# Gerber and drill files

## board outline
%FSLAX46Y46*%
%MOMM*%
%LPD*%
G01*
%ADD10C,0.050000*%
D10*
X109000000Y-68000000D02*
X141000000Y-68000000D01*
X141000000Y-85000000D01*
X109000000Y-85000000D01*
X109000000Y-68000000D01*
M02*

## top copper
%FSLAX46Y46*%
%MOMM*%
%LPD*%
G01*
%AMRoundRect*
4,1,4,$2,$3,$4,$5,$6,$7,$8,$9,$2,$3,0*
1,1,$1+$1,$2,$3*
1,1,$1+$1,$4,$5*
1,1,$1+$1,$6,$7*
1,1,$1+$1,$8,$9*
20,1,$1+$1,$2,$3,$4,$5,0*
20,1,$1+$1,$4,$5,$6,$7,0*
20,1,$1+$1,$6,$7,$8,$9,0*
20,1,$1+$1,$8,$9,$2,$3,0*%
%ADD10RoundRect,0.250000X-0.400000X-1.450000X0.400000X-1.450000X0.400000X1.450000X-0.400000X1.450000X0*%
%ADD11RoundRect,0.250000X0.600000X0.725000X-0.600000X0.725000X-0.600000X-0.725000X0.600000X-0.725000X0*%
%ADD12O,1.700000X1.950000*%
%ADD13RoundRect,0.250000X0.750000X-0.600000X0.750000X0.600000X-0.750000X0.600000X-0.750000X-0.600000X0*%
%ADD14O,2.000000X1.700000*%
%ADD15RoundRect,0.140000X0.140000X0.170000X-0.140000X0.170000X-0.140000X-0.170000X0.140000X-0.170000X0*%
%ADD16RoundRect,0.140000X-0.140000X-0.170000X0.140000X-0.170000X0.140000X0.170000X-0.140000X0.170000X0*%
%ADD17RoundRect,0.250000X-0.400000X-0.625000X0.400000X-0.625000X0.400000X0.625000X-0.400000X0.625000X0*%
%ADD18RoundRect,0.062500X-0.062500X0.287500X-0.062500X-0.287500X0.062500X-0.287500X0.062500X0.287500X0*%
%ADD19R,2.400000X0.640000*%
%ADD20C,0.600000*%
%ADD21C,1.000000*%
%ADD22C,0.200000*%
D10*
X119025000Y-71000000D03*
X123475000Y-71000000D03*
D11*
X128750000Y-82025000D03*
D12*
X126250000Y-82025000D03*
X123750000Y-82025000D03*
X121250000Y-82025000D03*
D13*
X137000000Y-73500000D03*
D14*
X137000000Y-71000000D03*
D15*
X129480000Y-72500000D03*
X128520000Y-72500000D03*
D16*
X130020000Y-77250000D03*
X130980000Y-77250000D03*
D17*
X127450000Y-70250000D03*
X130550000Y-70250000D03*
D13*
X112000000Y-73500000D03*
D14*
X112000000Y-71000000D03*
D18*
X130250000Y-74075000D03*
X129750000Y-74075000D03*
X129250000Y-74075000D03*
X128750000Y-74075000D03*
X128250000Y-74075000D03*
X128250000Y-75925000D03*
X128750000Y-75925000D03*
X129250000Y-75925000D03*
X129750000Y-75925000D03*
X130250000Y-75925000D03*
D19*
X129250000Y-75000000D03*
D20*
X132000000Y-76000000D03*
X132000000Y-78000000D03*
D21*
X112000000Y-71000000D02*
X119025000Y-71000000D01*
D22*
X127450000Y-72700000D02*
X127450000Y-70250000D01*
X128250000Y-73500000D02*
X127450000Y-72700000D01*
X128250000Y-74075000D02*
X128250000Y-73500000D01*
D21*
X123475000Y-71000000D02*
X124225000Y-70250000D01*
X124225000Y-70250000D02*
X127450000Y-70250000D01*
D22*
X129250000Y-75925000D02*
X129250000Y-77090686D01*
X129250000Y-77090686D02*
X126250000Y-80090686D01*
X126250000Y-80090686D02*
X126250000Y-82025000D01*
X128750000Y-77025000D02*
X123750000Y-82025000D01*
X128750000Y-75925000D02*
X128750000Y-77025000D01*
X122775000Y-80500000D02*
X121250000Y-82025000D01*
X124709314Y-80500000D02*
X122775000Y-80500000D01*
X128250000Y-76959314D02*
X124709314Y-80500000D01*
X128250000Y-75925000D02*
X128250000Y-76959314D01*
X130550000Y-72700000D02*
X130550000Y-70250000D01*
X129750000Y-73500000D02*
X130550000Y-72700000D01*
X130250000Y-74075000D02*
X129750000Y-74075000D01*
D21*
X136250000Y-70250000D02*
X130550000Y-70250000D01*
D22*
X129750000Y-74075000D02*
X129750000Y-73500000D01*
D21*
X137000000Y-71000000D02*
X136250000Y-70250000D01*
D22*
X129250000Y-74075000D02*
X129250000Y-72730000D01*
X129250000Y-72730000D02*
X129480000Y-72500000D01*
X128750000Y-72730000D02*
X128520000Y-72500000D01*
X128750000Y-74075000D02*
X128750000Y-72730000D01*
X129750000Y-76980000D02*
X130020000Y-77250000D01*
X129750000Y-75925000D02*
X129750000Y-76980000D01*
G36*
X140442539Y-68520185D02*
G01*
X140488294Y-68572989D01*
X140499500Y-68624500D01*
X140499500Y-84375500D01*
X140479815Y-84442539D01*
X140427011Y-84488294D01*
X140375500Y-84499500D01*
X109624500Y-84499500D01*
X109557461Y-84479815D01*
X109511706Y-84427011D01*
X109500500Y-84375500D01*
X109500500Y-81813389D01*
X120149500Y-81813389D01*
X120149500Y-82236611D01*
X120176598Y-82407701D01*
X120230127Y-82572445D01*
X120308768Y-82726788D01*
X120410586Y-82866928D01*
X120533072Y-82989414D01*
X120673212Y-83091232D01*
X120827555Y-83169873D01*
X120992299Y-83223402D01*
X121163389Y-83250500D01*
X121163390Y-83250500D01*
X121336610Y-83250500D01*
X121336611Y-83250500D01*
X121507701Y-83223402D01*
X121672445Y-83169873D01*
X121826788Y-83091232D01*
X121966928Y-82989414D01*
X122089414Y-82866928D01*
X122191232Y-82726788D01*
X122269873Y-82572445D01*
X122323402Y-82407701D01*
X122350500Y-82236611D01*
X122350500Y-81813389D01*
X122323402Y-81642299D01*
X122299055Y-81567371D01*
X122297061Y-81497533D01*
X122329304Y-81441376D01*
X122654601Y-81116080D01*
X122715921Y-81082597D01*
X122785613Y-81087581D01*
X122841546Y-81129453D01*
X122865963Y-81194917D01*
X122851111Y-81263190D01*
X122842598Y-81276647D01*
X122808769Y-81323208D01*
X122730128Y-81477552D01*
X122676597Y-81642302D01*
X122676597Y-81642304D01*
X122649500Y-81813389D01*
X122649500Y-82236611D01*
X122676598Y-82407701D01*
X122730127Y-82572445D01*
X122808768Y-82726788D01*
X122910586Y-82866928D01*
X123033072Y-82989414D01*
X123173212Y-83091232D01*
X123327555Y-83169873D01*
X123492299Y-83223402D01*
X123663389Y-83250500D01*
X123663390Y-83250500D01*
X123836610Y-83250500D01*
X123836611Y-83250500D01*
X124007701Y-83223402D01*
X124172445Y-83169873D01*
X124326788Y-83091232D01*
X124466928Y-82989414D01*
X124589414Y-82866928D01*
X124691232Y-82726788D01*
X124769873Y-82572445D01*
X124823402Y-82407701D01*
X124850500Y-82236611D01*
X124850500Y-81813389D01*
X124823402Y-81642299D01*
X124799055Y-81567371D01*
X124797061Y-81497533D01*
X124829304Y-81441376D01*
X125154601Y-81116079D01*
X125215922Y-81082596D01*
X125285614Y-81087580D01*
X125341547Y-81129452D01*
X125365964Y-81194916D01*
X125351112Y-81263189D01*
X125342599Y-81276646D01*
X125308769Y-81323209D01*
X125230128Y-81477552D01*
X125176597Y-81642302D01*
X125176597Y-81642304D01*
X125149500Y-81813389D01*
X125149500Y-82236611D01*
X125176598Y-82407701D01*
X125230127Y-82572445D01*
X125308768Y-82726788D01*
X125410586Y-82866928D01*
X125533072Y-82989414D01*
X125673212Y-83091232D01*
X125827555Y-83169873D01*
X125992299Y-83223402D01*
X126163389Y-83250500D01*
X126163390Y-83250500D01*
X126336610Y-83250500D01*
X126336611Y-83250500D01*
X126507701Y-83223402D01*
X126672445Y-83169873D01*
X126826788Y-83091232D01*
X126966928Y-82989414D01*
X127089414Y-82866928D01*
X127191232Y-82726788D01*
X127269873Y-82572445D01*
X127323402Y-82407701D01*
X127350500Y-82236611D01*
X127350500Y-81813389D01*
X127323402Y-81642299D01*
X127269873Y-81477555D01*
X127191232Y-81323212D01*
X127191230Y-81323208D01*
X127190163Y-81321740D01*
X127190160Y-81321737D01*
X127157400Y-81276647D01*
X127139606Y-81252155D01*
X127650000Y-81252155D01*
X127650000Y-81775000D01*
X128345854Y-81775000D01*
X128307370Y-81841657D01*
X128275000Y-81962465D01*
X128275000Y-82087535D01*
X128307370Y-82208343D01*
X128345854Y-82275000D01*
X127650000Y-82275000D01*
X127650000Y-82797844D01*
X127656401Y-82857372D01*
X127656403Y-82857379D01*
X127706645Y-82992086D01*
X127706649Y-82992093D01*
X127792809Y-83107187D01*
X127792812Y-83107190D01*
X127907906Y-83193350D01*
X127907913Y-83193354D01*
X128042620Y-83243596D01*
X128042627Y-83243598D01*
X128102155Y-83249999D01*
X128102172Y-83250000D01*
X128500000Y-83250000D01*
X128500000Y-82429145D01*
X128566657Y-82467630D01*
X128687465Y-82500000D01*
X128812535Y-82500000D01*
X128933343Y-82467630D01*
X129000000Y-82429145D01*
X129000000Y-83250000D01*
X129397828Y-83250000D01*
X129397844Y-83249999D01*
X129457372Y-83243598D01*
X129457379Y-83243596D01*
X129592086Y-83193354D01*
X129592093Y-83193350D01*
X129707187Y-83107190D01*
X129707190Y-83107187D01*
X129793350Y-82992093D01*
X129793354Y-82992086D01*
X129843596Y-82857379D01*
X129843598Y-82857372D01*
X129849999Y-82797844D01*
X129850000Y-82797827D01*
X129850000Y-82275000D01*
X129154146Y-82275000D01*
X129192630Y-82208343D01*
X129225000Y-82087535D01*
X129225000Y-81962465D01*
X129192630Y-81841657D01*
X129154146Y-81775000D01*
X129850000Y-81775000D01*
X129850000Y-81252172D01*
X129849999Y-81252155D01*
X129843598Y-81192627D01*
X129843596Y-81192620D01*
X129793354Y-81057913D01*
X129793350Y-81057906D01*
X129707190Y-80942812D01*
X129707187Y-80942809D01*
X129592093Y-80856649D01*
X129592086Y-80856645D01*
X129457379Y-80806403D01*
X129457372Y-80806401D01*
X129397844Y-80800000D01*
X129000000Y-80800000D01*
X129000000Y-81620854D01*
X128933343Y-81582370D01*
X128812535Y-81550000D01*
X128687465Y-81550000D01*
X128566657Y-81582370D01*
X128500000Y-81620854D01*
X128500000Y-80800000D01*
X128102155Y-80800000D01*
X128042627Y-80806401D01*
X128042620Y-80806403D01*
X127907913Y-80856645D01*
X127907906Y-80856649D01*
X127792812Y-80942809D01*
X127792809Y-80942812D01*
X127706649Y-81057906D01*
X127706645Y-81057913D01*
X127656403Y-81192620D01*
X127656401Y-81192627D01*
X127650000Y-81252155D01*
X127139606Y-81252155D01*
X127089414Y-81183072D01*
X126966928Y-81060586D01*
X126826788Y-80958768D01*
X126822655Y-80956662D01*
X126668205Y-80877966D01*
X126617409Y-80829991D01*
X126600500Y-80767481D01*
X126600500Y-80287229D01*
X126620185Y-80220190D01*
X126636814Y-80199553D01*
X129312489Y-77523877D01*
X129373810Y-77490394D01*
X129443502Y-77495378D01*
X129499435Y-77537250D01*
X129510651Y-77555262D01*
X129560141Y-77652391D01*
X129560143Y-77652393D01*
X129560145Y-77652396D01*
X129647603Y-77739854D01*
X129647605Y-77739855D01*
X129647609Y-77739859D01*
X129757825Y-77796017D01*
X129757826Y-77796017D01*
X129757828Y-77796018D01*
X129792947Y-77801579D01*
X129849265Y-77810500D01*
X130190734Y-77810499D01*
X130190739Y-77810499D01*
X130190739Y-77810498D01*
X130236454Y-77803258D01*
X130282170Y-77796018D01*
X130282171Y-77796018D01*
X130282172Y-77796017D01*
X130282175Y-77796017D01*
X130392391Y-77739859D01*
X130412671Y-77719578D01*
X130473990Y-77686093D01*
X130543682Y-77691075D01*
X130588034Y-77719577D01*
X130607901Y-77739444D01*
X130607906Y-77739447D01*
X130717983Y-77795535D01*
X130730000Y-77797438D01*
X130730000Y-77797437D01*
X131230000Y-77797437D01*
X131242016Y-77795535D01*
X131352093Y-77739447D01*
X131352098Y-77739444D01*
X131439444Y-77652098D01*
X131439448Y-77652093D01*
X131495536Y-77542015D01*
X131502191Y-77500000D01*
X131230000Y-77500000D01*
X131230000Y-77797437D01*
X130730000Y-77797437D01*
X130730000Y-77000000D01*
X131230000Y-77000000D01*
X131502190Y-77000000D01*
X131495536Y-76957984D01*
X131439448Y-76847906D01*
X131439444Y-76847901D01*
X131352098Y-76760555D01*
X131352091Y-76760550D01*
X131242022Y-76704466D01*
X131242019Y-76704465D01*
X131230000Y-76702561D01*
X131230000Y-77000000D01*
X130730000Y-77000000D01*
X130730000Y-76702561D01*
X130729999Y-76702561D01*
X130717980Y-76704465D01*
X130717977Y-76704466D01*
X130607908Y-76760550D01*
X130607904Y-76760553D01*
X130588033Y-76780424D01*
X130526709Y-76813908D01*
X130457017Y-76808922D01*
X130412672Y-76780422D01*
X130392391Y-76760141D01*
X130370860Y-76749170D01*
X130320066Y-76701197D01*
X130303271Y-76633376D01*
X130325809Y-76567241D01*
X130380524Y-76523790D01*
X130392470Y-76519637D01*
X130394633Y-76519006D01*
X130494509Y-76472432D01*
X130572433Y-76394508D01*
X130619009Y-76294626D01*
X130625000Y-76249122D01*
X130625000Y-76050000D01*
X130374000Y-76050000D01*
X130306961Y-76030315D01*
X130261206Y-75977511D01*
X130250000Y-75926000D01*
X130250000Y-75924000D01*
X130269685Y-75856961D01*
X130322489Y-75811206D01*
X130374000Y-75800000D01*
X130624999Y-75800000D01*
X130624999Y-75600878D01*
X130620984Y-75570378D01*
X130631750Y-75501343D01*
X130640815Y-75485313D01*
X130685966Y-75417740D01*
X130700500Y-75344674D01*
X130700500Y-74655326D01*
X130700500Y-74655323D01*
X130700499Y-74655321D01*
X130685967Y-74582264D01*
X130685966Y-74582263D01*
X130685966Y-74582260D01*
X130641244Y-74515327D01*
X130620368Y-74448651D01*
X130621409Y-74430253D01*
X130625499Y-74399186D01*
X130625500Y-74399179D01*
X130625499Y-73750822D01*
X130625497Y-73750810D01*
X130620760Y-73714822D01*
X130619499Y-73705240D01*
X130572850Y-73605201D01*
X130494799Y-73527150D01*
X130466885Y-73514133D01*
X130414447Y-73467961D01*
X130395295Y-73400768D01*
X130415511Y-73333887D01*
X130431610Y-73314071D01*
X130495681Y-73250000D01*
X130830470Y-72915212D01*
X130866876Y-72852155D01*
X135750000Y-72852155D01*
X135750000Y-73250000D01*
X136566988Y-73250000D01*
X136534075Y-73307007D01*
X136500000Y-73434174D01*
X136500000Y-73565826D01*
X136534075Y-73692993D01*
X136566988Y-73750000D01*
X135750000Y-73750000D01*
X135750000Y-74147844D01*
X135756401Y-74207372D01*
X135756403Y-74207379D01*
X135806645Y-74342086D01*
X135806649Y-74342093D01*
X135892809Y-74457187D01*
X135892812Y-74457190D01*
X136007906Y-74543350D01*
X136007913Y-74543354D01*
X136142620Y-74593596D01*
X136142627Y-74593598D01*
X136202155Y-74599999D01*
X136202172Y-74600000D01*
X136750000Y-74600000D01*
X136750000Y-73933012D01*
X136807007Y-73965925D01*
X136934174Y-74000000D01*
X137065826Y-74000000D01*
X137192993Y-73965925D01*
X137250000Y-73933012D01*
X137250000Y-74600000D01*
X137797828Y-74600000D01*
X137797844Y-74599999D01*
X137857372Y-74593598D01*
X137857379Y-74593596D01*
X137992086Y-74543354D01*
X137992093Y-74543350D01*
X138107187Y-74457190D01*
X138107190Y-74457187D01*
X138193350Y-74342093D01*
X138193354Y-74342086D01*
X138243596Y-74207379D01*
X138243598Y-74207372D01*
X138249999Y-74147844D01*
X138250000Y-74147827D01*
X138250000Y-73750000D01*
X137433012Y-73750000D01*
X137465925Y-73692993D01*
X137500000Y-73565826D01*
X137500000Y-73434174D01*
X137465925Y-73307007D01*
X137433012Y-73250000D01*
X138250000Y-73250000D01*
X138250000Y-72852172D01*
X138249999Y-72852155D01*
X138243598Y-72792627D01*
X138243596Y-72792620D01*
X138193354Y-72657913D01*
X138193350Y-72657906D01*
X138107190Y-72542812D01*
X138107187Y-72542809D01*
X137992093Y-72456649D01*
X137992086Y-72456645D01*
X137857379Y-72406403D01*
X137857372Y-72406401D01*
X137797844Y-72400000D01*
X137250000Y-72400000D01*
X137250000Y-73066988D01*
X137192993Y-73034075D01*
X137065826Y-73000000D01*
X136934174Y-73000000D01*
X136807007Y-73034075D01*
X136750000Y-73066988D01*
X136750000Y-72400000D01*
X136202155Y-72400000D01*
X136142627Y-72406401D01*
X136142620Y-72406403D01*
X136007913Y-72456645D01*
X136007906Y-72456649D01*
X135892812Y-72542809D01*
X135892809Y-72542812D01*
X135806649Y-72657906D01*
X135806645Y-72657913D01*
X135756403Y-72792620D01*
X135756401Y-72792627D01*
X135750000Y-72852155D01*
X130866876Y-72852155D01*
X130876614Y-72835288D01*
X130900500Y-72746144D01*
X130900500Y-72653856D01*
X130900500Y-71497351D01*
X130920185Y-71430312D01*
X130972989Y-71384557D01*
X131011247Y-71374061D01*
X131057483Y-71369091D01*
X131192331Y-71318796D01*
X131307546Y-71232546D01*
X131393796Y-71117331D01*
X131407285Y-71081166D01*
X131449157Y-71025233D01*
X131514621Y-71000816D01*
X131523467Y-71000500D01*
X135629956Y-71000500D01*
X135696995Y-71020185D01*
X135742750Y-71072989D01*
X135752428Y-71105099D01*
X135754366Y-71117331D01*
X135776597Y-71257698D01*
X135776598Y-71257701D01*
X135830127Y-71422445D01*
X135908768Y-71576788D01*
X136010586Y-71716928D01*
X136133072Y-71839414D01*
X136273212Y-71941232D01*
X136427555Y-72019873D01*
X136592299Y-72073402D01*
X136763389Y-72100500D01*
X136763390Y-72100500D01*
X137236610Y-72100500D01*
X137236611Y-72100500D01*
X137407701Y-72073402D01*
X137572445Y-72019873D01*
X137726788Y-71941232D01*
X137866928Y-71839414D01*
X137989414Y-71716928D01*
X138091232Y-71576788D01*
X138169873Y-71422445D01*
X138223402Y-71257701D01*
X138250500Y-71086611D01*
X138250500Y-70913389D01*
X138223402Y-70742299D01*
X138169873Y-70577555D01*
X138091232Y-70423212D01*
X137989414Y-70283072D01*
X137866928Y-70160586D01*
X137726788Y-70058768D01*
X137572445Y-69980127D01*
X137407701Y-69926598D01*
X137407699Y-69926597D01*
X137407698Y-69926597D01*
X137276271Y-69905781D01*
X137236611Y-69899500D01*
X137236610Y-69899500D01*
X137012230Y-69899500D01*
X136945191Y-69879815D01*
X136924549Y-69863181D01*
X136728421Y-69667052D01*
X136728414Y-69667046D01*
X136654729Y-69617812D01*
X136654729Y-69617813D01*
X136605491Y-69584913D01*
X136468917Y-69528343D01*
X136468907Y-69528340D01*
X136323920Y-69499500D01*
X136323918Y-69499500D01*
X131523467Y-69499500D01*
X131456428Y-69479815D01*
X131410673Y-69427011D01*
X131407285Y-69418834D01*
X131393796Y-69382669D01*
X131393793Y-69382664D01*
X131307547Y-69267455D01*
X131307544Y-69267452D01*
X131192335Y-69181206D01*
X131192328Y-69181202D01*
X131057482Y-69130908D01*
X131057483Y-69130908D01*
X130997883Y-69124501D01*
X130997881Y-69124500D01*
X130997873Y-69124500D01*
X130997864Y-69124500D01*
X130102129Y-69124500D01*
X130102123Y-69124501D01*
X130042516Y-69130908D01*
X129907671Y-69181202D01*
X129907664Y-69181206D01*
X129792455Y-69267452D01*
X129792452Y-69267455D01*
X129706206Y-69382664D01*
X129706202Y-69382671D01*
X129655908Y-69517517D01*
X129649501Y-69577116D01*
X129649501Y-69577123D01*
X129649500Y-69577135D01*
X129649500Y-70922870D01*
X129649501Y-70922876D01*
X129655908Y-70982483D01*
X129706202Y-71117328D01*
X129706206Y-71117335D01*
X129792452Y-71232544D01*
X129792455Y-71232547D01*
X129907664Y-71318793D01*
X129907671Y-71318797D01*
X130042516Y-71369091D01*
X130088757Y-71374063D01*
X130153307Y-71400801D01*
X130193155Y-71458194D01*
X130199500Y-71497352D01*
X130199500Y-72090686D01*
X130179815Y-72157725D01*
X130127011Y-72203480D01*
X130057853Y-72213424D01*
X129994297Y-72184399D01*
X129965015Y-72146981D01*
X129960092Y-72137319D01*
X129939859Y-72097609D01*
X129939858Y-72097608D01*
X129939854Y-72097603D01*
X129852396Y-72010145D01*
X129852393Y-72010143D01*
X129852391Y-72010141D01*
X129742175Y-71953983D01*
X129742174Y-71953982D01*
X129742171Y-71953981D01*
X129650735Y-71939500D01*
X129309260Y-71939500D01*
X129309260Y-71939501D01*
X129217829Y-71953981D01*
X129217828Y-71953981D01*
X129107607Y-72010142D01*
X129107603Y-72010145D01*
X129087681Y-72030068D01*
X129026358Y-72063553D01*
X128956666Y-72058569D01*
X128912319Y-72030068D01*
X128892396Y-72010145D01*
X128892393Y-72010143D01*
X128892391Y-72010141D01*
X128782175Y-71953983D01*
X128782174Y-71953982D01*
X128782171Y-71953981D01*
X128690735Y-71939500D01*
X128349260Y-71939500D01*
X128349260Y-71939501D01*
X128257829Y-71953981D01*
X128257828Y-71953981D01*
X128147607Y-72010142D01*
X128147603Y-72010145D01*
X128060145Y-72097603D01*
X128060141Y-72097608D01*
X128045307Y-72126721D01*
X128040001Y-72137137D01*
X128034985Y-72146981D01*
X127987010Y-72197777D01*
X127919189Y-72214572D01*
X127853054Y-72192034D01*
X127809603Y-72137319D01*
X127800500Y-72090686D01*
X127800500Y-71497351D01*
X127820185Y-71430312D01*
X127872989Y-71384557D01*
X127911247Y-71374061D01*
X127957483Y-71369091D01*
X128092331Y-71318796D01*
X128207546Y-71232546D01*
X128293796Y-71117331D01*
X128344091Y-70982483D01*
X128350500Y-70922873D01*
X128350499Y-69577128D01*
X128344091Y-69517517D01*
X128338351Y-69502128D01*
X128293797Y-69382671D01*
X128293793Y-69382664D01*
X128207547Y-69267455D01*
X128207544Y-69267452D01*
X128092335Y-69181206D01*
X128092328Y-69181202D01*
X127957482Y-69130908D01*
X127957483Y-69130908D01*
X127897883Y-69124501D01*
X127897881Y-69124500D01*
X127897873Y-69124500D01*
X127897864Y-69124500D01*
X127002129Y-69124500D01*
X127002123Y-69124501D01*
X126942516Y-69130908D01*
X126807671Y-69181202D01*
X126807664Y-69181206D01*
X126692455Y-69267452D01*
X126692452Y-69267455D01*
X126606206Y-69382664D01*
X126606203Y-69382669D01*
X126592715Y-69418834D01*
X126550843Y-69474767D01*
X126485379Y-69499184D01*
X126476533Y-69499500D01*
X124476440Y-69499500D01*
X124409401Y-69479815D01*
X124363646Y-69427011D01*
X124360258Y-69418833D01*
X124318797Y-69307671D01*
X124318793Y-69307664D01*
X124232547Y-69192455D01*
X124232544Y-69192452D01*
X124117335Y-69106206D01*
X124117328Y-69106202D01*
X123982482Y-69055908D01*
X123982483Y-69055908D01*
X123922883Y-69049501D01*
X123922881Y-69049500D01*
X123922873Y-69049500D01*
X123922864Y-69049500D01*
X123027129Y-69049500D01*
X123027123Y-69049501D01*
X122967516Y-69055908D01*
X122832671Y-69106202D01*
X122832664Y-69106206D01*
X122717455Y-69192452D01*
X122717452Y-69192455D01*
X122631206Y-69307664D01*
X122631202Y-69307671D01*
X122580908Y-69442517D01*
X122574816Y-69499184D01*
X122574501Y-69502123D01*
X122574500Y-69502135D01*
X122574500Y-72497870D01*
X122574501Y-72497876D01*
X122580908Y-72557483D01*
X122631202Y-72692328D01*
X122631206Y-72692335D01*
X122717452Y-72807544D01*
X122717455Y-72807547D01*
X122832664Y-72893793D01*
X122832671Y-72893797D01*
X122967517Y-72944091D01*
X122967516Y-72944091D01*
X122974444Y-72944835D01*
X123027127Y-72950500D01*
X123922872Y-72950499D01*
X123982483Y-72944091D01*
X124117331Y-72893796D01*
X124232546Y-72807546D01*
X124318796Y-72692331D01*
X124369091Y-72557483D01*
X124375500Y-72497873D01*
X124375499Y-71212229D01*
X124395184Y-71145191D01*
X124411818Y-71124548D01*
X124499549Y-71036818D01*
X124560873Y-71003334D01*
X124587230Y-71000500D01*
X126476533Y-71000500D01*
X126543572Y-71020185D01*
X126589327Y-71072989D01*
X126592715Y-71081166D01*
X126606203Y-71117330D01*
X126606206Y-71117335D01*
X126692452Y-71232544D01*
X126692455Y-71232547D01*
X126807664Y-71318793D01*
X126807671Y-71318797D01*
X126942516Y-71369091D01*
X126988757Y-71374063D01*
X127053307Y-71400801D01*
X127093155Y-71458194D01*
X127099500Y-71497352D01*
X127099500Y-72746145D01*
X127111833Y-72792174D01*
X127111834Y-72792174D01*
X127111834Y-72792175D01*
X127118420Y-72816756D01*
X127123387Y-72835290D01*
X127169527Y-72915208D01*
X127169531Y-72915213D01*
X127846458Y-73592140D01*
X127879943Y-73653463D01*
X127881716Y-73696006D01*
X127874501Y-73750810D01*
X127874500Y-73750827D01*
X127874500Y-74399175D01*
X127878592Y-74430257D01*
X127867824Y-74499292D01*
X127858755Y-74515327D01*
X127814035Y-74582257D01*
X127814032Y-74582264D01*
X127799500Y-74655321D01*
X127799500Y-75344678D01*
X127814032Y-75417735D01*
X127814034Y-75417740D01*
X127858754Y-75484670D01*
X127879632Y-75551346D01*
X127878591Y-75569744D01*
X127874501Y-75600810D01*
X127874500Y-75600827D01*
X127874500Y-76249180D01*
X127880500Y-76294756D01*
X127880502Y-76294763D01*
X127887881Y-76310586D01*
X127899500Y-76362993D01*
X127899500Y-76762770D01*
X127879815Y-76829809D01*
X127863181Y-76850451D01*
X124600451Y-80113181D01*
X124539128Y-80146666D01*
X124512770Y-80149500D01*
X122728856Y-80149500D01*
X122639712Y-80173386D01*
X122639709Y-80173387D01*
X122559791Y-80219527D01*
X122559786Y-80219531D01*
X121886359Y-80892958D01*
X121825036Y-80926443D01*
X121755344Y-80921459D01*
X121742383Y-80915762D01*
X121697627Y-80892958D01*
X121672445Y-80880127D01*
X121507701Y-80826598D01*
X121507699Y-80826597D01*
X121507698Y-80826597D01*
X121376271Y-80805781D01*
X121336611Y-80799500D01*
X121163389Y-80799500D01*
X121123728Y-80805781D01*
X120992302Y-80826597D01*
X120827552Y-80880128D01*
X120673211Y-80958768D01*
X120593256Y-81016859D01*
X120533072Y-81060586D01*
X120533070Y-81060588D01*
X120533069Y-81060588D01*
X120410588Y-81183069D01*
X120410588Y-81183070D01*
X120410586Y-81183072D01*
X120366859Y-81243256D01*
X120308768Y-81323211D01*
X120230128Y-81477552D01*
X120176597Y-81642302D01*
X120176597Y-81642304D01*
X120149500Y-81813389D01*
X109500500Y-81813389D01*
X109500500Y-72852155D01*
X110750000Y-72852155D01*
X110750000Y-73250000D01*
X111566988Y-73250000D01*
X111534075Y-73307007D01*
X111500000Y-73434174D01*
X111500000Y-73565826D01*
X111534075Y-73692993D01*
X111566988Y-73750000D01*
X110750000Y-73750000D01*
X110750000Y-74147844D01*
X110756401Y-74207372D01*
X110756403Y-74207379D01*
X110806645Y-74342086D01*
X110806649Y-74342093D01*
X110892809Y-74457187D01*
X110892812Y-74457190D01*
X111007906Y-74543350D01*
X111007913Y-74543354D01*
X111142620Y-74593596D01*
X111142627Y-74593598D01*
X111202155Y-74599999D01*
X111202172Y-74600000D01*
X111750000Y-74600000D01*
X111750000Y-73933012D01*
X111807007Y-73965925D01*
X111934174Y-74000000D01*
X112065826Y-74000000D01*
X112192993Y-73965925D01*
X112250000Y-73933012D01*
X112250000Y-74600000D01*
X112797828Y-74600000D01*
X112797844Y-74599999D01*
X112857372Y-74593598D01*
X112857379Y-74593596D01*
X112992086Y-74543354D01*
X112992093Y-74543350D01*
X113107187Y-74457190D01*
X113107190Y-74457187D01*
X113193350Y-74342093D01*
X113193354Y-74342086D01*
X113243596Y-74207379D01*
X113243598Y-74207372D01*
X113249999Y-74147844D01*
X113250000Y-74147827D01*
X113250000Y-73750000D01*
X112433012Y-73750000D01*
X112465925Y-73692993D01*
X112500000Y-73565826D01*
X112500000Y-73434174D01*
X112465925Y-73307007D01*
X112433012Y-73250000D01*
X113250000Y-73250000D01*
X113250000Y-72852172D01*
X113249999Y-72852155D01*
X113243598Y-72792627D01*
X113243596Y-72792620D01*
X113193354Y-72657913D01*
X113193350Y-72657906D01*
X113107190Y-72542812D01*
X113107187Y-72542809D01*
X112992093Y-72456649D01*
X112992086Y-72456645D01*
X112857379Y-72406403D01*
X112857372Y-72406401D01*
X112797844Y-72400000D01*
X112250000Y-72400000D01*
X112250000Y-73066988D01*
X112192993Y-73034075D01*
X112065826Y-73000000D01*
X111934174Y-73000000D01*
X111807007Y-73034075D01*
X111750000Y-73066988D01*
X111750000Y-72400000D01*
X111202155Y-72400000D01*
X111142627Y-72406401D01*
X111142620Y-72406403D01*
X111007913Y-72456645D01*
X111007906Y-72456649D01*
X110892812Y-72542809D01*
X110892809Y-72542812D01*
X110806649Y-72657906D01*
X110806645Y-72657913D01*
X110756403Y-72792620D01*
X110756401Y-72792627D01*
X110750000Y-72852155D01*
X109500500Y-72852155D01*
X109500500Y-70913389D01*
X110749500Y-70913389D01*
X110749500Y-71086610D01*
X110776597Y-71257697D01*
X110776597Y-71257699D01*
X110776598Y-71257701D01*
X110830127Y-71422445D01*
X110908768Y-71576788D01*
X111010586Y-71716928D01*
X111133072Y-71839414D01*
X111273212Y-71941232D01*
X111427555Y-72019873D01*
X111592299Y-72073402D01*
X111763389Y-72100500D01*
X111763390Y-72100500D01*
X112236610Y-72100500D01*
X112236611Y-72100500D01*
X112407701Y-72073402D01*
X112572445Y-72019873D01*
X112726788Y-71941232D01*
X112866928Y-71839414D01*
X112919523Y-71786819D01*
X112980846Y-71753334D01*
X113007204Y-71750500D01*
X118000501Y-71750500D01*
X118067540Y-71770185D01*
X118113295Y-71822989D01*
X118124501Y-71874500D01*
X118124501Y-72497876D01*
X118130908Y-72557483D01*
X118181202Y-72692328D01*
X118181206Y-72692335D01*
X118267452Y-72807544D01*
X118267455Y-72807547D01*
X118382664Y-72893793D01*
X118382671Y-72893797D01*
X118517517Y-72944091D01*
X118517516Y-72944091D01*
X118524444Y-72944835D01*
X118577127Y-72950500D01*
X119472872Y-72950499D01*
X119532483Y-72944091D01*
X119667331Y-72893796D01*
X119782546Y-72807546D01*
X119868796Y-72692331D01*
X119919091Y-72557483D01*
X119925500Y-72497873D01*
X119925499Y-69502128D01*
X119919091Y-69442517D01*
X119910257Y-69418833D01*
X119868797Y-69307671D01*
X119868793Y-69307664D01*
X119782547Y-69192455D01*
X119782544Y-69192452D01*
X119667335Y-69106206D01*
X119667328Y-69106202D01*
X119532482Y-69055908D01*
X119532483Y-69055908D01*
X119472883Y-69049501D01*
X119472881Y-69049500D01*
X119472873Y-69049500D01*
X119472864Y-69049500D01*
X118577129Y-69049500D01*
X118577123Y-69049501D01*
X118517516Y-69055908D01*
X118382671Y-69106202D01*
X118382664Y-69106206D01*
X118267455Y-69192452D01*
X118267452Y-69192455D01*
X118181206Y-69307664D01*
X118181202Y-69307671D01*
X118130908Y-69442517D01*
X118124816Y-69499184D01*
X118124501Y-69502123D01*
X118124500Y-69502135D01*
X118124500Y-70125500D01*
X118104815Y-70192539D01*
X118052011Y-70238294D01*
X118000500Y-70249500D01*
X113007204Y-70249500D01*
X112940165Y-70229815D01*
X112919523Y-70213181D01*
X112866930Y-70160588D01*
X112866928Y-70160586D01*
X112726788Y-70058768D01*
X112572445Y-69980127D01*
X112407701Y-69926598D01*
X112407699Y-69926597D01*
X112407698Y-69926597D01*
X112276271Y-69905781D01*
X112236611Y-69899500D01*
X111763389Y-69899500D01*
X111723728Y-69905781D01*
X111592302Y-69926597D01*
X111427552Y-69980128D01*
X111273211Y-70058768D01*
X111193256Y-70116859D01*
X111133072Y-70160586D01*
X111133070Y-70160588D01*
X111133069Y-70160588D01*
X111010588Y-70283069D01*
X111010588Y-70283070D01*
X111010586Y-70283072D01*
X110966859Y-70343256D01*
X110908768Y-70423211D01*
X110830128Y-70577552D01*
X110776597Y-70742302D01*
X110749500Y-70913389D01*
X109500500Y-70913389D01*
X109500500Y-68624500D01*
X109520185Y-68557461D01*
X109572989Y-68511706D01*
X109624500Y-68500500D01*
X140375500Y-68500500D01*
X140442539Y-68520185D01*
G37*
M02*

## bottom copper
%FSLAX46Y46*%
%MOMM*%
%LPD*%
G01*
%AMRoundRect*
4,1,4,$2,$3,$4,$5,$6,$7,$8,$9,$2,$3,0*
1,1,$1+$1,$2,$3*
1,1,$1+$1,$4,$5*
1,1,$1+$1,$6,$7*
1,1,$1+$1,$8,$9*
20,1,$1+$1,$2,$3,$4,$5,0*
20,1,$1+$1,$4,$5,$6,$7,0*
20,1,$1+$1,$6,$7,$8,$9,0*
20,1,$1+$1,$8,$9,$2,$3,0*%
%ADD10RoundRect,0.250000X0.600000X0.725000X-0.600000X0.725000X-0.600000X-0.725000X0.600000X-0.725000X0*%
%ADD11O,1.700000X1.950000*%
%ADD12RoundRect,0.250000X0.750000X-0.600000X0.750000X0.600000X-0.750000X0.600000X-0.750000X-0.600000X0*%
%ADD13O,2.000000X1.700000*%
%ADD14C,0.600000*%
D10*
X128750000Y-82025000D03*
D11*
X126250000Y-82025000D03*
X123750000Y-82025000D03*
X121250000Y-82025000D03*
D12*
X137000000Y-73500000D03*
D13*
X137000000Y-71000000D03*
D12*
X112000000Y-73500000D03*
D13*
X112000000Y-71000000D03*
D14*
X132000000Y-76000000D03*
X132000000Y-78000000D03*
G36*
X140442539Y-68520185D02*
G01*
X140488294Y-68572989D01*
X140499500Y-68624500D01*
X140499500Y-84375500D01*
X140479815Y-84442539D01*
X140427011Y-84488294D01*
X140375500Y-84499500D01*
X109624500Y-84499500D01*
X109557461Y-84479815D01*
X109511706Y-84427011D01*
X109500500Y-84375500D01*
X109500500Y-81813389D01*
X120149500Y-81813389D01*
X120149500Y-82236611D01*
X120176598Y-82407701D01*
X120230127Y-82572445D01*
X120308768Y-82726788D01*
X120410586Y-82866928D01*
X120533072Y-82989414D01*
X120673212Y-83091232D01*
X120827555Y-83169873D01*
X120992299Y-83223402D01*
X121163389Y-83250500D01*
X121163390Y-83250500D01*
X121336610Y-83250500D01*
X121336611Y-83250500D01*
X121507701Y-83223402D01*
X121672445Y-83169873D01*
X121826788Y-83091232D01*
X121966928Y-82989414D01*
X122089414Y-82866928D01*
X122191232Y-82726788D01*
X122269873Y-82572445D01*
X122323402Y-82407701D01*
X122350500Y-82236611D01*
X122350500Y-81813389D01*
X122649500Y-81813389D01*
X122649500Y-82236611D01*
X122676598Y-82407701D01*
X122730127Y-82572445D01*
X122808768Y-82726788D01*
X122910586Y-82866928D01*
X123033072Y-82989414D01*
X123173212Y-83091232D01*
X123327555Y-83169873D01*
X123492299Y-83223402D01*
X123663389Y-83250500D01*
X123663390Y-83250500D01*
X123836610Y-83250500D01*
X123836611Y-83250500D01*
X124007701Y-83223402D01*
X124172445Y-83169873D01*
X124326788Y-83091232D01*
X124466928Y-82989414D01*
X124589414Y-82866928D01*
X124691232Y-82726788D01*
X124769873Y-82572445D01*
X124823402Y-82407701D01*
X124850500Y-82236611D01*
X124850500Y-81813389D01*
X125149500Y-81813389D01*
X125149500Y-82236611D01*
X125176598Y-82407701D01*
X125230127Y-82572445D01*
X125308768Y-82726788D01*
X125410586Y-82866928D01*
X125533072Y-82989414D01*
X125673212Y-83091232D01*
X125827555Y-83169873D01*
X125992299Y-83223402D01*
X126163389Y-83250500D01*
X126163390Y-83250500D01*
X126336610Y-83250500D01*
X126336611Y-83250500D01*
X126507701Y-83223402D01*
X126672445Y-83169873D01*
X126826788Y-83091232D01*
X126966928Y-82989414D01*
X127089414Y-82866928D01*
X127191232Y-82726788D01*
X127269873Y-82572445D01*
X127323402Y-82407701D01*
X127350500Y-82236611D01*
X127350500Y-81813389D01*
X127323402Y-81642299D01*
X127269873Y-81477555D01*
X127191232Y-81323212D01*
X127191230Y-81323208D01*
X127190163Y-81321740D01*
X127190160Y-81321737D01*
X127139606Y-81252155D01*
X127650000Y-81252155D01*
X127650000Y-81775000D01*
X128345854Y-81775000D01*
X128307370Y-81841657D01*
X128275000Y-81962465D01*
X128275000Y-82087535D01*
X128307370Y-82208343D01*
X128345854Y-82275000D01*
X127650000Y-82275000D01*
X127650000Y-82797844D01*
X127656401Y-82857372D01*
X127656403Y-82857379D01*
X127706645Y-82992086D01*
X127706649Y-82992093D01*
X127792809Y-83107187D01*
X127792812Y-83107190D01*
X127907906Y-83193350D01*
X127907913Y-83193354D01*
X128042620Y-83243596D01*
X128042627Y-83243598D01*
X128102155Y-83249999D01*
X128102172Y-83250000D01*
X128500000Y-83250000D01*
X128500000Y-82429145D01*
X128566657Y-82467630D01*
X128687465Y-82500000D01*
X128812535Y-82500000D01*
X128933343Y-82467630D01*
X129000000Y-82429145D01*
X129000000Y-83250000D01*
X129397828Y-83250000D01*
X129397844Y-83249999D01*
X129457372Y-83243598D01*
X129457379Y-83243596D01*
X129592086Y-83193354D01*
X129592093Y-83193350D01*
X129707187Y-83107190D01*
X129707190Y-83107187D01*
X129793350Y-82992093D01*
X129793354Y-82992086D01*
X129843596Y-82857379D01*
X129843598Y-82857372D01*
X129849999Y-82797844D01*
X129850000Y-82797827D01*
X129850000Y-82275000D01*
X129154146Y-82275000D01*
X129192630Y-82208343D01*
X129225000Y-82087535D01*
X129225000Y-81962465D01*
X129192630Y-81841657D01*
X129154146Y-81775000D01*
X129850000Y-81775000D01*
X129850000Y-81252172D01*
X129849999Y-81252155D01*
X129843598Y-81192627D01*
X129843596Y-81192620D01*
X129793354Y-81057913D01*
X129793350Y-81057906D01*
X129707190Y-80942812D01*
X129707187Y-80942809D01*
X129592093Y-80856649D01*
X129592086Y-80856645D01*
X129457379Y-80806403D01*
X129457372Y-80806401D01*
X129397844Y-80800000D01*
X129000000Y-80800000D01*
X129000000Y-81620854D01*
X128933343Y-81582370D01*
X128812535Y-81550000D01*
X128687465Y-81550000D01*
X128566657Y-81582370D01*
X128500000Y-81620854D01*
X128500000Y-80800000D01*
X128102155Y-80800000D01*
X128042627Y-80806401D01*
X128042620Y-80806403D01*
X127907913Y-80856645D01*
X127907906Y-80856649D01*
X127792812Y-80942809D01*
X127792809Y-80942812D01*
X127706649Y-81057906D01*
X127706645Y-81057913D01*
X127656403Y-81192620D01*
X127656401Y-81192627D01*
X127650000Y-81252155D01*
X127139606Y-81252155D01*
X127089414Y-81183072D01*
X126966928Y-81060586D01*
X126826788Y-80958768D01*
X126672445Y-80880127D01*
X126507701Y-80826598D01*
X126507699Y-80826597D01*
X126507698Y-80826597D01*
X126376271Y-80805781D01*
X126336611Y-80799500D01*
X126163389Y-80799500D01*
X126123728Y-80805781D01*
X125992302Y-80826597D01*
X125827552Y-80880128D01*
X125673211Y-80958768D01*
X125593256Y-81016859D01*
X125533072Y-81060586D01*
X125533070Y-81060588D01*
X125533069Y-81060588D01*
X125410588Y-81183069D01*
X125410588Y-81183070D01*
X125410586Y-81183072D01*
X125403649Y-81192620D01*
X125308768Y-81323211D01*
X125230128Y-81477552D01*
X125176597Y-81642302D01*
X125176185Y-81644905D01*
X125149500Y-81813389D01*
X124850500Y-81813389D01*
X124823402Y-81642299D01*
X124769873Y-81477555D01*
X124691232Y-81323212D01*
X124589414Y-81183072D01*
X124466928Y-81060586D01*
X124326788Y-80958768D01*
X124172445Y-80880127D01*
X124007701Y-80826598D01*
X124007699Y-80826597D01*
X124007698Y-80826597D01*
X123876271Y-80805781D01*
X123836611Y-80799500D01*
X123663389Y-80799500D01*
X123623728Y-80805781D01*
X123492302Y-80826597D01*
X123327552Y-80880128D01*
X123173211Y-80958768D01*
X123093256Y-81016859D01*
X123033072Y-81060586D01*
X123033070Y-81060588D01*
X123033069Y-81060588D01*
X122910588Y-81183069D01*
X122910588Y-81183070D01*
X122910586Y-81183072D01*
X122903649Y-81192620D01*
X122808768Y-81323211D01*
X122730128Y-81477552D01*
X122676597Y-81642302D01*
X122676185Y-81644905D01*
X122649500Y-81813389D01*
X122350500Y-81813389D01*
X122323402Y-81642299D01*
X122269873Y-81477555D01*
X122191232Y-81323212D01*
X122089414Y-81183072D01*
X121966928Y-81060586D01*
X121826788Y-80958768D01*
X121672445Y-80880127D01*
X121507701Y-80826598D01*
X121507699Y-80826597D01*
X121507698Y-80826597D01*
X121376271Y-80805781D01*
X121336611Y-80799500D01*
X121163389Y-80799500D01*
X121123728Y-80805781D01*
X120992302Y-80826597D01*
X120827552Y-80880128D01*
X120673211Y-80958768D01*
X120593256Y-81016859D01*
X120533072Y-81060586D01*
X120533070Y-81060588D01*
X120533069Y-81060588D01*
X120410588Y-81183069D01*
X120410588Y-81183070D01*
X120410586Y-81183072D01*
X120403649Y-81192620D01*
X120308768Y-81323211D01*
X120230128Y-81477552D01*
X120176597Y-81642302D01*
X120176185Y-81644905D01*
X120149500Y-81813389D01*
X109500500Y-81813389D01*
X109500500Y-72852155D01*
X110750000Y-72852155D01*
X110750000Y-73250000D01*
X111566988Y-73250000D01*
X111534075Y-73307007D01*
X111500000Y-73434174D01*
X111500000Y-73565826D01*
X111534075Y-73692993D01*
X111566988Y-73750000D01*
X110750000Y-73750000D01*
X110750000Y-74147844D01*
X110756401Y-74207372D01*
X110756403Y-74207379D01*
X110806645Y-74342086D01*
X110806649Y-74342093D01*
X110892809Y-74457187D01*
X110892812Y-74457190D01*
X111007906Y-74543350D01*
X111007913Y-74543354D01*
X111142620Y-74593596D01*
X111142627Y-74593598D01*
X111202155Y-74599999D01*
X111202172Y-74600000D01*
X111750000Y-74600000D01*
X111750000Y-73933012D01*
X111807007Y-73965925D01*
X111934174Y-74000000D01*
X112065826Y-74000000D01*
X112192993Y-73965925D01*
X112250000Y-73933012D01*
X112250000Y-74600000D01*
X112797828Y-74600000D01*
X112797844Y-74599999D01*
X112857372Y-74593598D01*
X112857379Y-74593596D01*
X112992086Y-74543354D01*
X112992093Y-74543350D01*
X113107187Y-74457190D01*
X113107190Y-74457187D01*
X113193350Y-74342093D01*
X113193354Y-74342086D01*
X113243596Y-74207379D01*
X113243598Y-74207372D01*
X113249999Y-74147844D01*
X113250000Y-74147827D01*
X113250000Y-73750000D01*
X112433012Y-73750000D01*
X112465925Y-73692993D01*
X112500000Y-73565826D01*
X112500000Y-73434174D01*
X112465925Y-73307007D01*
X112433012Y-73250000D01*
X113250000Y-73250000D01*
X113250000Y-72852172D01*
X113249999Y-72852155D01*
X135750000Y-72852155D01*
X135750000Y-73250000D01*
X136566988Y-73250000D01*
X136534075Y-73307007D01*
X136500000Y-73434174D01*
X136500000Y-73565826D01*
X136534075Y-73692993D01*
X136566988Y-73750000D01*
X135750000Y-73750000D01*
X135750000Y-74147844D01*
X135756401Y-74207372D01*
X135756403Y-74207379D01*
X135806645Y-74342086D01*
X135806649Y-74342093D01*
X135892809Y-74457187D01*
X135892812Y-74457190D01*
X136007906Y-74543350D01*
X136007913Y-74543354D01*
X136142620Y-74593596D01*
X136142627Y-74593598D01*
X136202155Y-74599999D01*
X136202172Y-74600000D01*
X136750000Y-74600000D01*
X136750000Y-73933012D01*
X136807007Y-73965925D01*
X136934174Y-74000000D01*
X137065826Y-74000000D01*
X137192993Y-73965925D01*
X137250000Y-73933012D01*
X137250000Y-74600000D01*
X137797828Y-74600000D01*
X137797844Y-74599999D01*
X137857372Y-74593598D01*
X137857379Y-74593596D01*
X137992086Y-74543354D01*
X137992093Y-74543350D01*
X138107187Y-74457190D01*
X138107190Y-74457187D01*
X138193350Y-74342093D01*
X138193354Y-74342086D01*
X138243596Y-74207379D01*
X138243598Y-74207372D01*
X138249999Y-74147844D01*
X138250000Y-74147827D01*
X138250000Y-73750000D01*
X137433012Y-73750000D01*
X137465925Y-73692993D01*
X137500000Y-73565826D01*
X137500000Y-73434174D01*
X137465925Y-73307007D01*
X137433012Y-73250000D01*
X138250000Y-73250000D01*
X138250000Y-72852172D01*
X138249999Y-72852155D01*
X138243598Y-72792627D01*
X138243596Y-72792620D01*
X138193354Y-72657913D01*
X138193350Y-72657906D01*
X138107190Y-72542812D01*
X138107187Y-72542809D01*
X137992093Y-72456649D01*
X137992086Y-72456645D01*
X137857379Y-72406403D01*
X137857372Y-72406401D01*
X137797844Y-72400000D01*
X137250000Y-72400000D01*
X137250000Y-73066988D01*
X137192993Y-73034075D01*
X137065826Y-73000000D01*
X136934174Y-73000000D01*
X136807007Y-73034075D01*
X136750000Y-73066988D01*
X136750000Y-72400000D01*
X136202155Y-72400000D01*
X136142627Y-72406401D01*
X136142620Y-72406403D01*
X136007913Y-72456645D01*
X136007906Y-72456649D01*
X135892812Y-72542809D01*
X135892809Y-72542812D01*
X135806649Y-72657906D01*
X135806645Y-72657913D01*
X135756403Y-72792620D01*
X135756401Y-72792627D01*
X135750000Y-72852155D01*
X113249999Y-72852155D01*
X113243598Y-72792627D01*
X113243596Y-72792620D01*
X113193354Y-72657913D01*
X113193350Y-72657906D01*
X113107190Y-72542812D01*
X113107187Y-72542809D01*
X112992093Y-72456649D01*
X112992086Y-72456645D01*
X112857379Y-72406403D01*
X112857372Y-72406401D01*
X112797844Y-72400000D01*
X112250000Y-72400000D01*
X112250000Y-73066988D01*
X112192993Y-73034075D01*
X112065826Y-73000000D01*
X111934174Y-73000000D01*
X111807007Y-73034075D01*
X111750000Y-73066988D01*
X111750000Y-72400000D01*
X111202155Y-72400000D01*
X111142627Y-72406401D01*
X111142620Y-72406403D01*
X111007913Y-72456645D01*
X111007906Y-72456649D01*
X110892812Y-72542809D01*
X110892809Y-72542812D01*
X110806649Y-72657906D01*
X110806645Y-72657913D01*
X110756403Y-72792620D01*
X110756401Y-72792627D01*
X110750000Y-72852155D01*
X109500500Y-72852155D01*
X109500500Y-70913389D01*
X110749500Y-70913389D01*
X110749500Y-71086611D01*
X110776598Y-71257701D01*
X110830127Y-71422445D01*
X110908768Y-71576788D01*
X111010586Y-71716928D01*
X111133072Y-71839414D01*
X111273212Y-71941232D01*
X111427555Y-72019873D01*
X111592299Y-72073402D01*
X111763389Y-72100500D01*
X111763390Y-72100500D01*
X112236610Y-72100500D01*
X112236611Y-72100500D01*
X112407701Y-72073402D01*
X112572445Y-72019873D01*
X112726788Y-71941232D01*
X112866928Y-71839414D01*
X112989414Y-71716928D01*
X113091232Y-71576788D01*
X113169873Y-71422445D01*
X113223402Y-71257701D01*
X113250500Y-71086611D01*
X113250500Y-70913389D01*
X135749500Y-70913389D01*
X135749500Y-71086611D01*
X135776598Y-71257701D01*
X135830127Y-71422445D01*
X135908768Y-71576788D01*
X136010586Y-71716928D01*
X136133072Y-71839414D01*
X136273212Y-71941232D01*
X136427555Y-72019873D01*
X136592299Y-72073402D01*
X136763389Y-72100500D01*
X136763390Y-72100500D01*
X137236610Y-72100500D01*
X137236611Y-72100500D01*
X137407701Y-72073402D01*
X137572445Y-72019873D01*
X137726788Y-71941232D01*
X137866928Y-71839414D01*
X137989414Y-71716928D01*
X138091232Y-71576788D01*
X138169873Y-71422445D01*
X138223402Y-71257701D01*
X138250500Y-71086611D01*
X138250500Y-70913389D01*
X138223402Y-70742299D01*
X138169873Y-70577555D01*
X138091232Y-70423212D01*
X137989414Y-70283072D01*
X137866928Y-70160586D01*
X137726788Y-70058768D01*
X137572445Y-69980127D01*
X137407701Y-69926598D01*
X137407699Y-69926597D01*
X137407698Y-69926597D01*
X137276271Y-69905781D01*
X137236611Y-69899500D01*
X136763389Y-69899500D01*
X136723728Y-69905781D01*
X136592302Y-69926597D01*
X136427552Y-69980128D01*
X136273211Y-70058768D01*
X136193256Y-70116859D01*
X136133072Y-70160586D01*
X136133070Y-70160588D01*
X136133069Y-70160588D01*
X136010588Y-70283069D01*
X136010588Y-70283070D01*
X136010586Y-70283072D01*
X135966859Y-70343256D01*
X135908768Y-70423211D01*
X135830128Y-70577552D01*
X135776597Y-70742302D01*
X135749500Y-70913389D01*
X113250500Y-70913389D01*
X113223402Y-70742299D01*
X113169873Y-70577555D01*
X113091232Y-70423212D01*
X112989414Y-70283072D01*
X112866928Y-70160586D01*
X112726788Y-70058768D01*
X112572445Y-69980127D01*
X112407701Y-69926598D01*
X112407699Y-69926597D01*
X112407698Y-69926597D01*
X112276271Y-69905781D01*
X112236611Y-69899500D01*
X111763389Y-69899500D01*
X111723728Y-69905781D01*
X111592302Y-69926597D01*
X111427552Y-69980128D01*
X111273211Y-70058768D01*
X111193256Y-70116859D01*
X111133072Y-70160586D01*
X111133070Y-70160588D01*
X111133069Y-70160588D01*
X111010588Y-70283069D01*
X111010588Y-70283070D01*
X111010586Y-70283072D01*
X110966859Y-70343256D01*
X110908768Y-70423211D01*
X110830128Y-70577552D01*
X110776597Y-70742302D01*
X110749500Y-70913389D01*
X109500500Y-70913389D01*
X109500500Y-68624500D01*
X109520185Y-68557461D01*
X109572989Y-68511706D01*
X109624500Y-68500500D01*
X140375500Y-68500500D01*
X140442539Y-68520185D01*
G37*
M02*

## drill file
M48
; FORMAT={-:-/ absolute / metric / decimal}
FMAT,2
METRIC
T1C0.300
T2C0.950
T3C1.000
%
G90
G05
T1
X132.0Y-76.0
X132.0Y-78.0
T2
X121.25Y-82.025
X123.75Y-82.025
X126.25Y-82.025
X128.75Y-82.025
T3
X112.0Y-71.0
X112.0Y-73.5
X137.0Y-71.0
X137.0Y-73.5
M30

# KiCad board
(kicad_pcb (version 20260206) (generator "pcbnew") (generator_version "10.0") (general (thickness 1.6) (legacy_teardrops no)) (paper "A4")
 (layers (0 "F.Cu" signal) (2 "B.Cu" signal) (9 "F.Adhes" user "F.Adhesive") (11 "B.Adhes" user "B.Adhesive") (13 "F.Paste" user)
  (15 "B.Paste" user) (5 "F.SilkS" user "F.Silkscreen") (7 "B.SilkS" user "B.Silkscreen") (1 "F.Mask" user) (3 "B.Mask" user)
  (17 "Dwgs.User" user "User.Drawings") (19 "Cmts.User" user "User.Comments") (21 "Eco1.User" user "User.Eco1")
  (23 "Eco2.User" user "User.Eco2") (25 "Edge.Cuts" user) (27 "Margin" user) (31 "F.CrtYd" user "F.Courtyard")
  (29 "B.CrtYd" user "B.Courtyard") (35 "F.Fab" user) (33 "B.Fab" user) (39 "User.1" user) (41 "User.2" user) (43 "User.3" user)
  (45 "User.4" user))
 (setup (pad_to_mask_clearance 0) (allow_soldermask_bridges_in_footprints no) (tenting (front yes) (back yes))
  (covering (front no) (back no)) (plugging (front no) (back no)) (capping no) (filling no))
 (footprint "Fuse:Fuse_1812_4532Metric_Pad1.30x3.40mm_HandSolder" (layer "F.Cu") (at 121.25 71)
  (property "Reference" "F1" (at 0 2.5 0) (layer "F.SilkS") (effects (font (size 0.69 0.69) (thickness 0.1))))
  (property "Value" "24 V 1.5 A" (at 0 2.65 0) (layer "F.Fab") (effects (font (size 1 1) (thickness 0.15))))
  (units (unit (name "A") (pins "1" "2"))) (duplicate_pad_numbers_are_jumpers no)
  (pad "1" smd roundrect (at -2.225 0) (size 1.3 3.4) (layers "F.Cu" "F.Mask" "F.Paste") (roundrect_rratio 0.192308) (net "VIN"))
  (pad "2" smd roundrect (at 2.225 0) (size 1.3 3.4) (layers "F.Cu" "F.Mask" "F.Paste") (roundrect_rratio 0.192308) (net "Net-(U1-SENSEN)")))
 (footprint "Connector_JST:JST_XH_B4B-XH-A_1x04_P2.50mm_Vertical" (layer "F.Cu") (at 128.75 82.025 180)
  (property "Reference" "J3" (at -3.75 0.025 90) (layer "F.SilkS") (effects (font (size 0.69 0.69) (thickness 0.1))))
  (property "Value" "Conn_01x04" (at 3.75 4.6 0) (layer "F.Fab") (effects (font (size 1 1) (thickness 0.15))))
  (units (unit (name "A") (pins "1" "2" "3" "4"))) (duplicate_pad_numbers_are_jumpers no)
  (pad "1" thru_hole roundrect (at 0 0 180) (size 1.7 1.95) (drill 0.95) (layers "*.Cu" "*.Mask") (remove_unused_layers no)
   (roundrect_rratio 0.147059) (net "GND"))
  (pad "2" thru_hole oval (at 2.5 0 180) (size 1.7 1.95) (drill 0.95) (layers "*.Cu" "*.Mask") (remove_unused_layers no) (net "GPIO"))
  (pad "3" thru_hole oval (at 5 0 180) (size 1.7 1.95) (drill 0.95) (layers "*.Cu" "*.Mask") (remove_unused_layers no) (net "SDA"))
  (pad "4" thru_hole oval (at 7.5 0 180) (size 1.7 1.95) (drill 0.95) (layers "*.Cu" "*.Mask") (remove_unused_layers no) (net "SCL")))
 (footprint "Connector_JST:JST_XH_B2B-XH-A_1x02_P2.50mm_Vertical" (layer "F.Cu") (at 137 73.5 90)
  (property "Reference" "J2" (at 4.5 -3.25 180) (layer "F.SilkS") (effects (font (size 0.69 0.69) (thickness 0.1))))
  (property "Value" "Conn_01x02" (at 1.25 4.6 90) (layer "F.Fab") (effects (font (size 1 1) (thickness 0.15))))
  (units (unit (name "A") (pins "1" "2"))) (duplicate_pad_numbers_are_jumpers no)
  (pad "1" thru_hole roundrect (at 0 0 90) (size 1.7 2) (drill 1) (layers "*.Cu" "*.Mask") (remove_unused_layers no)
   (roundrect_rratio 0.147059) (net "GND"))
  (pad "2" thru_hole oval (at 2.5 0 90) (size 1.7 2) (drill 1) (layers "*.Cu" "*.Mask") (remove_unused_layers no) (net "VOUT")))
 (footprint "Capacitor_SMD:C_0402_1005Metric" (layer "F.Cu") (at 129 72.5 180)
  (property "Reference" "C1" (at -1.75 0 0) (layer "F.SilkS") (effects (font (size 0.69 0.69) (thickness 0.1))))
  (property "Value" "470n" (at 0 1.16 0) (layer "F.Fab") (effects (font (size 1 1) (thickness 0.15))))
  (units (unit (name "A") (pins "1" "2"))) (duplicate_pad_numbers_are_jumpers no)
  (pad "1" smd roundrect (at -0.48 0 180) (size 0.56 0.62) (layers "F.Cu" "F.Mask" "F.Paste") (roundrect_rratio 0.25) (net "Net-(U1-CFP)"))
  (pad "2" smd roundrect (at 0.48 0 180) (size 0.56 0.62) (layers "F.Cu" "F.Mask" "F.Paste") (roundrect_rratio 0.25) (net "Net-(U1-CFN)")))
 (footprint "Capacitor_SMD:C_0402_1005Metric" (layer "F.Cu") (at 130.5 77.25)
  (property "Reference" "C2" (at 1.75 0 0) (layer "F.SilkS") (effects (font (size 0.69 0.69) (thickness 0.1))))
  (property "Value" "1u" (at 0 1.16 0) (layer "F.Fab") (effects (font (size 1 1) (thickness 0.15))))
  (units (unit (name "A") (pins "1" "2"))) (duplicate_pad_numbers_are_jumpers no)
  (pad "1" smd roundrect (at -0.48 0) (size 0.56 0.62) (layers "F.Cu" "F.Mask" "F.Paste") (roundrect_rratio 0.25) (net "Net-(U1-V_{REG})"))
  (pad "2" smd roundrect (at 0.48 0) (size 0.56 0.62) (layers "F.Cu" "F.Mask" "F.Paste") (roundrect_rratio 0.25) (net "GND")))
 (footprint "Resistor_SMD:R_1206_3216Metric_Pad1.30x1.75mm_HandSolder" (layer "F.Cu") (at 129 70.25)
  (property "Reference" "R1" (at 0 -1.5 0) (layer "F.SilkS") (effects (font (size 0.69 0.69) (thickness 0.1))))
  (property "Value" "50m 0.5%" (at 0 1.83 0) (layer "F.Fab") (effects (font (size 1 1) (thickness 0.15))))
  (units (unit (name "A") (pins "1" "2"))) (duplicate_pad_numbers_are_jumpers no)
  (pad "1" smd roundrect (at -1.55 0) (size 1.3 1.75) (layers "F.Cu" "F.Mask" "F.Paste") (roundrect_rratio 0.192308) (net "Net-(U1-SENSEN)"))
  (pad "2" smd roundrect (at 1.55 0) (size 1.3 1.75) (layers "F.Cu" "F.Mask" "F.Paste") (roundrect_rratio 0.192308) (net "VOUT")))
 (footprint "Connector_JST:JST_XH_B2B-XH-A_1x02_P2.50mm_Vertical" (layer "F.Cu") (at 112 73.5 90)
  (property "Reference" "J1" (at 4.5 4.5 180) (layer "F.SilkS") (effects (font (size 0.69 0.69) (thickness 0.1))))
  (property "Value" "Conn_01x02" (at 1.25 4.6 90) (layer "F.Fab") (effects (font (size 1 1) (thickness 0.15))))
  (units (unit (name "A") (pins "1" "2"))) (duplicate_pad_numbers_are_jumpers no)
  (pad "1" thru_hole roundrect (at 0 0 90) (size 1.7 2) (drill 1) (layers "*.Cu" "*.Mask") (remove_unused_layers no)
   (roundrect_rratio 0.147059) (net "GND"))
  (pad "2" thru_hole oval (at 2.5 0 90) (size 1.7 2) (drill 1) (layers "*.Cu" "*.Mask") (remove_unused_layers no) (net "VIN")))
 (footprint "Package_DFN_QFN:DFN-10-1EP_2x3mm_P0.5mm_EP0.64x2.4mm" (layer "F.Cu") (at 129.25 75 -90)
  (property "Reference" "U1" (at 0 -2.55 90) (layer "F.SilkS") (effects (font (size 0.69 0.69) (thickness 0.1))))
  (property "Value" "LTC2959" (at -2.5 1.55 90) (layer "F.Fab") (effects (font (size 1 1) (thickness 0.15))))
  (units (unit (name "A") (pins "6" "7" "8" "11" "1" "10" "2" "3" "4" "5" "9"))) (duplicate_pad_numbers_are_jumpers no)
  (pad "" smd roundrect (at 0 -0.6 270) (size 0.5 1) (layers "F.Paste") (roundrect_rratio 0.25))
  (pad "" smd roundrect (at 0 0.6 270) (size 0.5 1) (layers "F.Paste") (roundrect_rratio 0.25))
  (pad "1" smd roundrect (at -0.925 -1 270) (size 0.7 0.25) (layers "F.Cu" "F.Mask" "F.Paste") (roundrect_rratio 0.25) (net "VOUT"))
  (pad "2" smd roundrect (at -0.925 -0.5 270) (size 0.7 0.25) (layers "F.Cu" "F.Mask" "F.Paste") (roundrect_rratio 0.25) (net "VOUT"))
  (pad "3" smd roundrect (at -0.925 0 270) (size 0.7 0.25) (layers "F.Cu" "F.Mask" "F.Paste") (roundrect_rratio 0.25) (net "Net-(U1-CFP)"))
  (pad "4" smd roundrect (at -0.925 0.5 270) (size 0.7 0.25) (layers "F.Cu" "F.Mask" "F.Paste") (roundrect_rratio 0.25) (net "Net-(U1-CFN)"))
  (pad "5" smd roundrect (at -0.925 1 270) (size 0.7 0.25) (layers "F.Cu" "F.Mask" "F.Paste") (roundrect_rratio 0.25)
   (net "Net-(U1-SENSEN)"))
  (pad "6" smd roundrect (at 0.925 1 270) (size 0.7 0.25) (layers "F.Cu" "F.Mask" "F.Paste") (roundrect_rratio 0.25) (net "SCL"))
  (pad "7" smd roundrect (at 0.925 0.5 270) (size 0.7 0.25) (layers "F.Cu" "F.Mask" "F.Paste") (roundrect_rratio 0.25) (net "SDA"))
  (pad "8" smd roundrect (at 0.925 0 270) (size 0.7 0.25) (layers "F.Cu" "F.Mask" "F.Paste") (roundrect_rratio 0.25) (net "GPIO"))
  (pad "9" smd roundrect (at 0.925 -0.5 270) (size 0.7 0.25) (layers "F.Cu" "F.Mask" "F.Paste") (roundrect_rratio 0.25)
   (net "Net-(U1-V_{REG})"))
  (pad "10" smd roundrect (at 0.925 -1 270) (size 0.7 0.25) (layers "F.Cu" "F.Mask" "F.Paste") (roundrect_rratio 0.25) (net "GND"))
  (pad "11" smd rect (at 0 0 270) (size 0.64 2.4) (layers "F.Cu" "F.Mask") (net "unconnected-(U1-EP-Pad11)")
   (solder_paste_margin_ratio -0.2)))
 (gr_rect (start 109 68) (end 141 85) (stroke (width 0.05) (type default)) (fill no) (layer "Edge.Cuts"))
 (segment (start 112 71) (end 119.025 71) (width 1) (layer "F.Cu") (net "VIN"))
 (segment (start 127.45 72.7) (end 127.45 70.25) (width 0.2) (layer "F.Cu") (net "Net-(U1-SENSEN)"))
 (segment (start 128.25 73.5) (end 127.45 72.7) (width 0.2) (layer "F.Cu") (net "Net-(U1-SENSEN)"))
 (segment (start 128.25 74.075) (end 128.25 73.5) (width 0.2) (layer "F.Cu") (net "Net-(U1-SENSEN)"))
 (segment (start 123.475 71) (end 124.225 70.25) (width 1) (layer "F.Cu") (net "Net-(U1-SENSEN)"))
 (segment (start 124.225 70.25) (end 127.45 70.25) (width 1) (layer "F.Cu") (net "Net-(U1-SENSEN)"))
 (via (at 132 76) (size 0.6) (drill 0.3) (layers "F.Cu" "B.Cu") (free yes) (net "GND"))
 (via (at 132 78) (size 0.6) (drill 0.3) (layers "F.Cu" "B.Cu") (free yes) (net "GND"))
 (segment (start 129.25 75.925) (end 129.25 77.090686) (width 0.2) (layer "F.Cu") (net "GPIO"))
 (segment (start 129.25 77.090686) (end 126.25 80.090686) (width 0.2) (layer "F.Cu") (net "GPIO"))
 (segment (start 126.25 80.090686) (end 126.25 82.025) (width 0.2) (layer "F.Cu") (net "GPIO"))
 (segment (start 128.75 77.025) (end 123.75 82.025) (width 0.2) (layer "F.Cu") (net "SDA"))
 (segment (start 128.75 75.925) (end 128.75 77.025) (width 0.2) (layer "F.Cu") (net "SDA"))
 (segment (start 122.775 80.5) (end 121.25 82.025) (width 0.2) (layer "F.Cu") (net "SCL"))
 (segment (start 124.709314 80.5) (end 122.775 80.5) (width 0.2) (layer "F.Cu") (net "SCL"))
 (segment (start 128.25 76.959314) (end 124.709314 80.5) (width 0.2) (layer "F.Cu") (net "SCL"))
 (segment (start 128.25 75.925) (end 128.25 76.959314) (width 0.2) (layer "F.Cu") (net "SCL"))
 (segment (start 130.55 72.7) (end 130.55 70.25) (width 0.2) (layer "F.Cu") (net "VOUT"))
 (segment (start 129.75 73.5) (end 130.55 72.7) (width 0.2) (layer "F.Cu") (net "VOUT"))
 (segment (start 130.25 74.075) (end 129.75 74.075) (width 0.2) (layer "F.Cu") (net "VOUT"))
 (segment (start 136.25 70.25) (end 130.55 70.25) (width 1) (layer "F.Cu") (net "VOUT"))
 (segment (start 129.75 74.075) (end 129.75 73.5) (width 0.2) (layer "F.Cu") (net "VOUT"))
 (segment (start 137 71) (end 136.25 70.25) (width 1) (layer "F.Cu") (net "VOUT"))
 (segment (start 129.25 74.075) (end 129.25 72.73) (width 0.2) (layer "F.Cu") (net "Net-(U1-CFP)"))
 (segment (start 129.25 72.73) (end 129.48 72.5) (width 0.2) (layer "F.Cu") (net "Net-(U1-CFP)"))
 (segment (start 128.75 72.73) (end 128.52 72.5) (width 0.2) (layer "F.Cu") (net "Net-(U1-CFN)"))
 (segment (start 128.75 74.075) (end 128.75 72.73) (width 0.2) (layer "F.Cu") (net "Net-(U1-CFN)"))
 (segment (start 129.75 76.98) (end 130.02 77.25) (width 0.2) (layer "F.Cu") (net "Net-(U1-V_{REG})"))
 (segment (start 129.75 75.925) (end 129.75 76.98) (width 0.2) (layer "F.Cu") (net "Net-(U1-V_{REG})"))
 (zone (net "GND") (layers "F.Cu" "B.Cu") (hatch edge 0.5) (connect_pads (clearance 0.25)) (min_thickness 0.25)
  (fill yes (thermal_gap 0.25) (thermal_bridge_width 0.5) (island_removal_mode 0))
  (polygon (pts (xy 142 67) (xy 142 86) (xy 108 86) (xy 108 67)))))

